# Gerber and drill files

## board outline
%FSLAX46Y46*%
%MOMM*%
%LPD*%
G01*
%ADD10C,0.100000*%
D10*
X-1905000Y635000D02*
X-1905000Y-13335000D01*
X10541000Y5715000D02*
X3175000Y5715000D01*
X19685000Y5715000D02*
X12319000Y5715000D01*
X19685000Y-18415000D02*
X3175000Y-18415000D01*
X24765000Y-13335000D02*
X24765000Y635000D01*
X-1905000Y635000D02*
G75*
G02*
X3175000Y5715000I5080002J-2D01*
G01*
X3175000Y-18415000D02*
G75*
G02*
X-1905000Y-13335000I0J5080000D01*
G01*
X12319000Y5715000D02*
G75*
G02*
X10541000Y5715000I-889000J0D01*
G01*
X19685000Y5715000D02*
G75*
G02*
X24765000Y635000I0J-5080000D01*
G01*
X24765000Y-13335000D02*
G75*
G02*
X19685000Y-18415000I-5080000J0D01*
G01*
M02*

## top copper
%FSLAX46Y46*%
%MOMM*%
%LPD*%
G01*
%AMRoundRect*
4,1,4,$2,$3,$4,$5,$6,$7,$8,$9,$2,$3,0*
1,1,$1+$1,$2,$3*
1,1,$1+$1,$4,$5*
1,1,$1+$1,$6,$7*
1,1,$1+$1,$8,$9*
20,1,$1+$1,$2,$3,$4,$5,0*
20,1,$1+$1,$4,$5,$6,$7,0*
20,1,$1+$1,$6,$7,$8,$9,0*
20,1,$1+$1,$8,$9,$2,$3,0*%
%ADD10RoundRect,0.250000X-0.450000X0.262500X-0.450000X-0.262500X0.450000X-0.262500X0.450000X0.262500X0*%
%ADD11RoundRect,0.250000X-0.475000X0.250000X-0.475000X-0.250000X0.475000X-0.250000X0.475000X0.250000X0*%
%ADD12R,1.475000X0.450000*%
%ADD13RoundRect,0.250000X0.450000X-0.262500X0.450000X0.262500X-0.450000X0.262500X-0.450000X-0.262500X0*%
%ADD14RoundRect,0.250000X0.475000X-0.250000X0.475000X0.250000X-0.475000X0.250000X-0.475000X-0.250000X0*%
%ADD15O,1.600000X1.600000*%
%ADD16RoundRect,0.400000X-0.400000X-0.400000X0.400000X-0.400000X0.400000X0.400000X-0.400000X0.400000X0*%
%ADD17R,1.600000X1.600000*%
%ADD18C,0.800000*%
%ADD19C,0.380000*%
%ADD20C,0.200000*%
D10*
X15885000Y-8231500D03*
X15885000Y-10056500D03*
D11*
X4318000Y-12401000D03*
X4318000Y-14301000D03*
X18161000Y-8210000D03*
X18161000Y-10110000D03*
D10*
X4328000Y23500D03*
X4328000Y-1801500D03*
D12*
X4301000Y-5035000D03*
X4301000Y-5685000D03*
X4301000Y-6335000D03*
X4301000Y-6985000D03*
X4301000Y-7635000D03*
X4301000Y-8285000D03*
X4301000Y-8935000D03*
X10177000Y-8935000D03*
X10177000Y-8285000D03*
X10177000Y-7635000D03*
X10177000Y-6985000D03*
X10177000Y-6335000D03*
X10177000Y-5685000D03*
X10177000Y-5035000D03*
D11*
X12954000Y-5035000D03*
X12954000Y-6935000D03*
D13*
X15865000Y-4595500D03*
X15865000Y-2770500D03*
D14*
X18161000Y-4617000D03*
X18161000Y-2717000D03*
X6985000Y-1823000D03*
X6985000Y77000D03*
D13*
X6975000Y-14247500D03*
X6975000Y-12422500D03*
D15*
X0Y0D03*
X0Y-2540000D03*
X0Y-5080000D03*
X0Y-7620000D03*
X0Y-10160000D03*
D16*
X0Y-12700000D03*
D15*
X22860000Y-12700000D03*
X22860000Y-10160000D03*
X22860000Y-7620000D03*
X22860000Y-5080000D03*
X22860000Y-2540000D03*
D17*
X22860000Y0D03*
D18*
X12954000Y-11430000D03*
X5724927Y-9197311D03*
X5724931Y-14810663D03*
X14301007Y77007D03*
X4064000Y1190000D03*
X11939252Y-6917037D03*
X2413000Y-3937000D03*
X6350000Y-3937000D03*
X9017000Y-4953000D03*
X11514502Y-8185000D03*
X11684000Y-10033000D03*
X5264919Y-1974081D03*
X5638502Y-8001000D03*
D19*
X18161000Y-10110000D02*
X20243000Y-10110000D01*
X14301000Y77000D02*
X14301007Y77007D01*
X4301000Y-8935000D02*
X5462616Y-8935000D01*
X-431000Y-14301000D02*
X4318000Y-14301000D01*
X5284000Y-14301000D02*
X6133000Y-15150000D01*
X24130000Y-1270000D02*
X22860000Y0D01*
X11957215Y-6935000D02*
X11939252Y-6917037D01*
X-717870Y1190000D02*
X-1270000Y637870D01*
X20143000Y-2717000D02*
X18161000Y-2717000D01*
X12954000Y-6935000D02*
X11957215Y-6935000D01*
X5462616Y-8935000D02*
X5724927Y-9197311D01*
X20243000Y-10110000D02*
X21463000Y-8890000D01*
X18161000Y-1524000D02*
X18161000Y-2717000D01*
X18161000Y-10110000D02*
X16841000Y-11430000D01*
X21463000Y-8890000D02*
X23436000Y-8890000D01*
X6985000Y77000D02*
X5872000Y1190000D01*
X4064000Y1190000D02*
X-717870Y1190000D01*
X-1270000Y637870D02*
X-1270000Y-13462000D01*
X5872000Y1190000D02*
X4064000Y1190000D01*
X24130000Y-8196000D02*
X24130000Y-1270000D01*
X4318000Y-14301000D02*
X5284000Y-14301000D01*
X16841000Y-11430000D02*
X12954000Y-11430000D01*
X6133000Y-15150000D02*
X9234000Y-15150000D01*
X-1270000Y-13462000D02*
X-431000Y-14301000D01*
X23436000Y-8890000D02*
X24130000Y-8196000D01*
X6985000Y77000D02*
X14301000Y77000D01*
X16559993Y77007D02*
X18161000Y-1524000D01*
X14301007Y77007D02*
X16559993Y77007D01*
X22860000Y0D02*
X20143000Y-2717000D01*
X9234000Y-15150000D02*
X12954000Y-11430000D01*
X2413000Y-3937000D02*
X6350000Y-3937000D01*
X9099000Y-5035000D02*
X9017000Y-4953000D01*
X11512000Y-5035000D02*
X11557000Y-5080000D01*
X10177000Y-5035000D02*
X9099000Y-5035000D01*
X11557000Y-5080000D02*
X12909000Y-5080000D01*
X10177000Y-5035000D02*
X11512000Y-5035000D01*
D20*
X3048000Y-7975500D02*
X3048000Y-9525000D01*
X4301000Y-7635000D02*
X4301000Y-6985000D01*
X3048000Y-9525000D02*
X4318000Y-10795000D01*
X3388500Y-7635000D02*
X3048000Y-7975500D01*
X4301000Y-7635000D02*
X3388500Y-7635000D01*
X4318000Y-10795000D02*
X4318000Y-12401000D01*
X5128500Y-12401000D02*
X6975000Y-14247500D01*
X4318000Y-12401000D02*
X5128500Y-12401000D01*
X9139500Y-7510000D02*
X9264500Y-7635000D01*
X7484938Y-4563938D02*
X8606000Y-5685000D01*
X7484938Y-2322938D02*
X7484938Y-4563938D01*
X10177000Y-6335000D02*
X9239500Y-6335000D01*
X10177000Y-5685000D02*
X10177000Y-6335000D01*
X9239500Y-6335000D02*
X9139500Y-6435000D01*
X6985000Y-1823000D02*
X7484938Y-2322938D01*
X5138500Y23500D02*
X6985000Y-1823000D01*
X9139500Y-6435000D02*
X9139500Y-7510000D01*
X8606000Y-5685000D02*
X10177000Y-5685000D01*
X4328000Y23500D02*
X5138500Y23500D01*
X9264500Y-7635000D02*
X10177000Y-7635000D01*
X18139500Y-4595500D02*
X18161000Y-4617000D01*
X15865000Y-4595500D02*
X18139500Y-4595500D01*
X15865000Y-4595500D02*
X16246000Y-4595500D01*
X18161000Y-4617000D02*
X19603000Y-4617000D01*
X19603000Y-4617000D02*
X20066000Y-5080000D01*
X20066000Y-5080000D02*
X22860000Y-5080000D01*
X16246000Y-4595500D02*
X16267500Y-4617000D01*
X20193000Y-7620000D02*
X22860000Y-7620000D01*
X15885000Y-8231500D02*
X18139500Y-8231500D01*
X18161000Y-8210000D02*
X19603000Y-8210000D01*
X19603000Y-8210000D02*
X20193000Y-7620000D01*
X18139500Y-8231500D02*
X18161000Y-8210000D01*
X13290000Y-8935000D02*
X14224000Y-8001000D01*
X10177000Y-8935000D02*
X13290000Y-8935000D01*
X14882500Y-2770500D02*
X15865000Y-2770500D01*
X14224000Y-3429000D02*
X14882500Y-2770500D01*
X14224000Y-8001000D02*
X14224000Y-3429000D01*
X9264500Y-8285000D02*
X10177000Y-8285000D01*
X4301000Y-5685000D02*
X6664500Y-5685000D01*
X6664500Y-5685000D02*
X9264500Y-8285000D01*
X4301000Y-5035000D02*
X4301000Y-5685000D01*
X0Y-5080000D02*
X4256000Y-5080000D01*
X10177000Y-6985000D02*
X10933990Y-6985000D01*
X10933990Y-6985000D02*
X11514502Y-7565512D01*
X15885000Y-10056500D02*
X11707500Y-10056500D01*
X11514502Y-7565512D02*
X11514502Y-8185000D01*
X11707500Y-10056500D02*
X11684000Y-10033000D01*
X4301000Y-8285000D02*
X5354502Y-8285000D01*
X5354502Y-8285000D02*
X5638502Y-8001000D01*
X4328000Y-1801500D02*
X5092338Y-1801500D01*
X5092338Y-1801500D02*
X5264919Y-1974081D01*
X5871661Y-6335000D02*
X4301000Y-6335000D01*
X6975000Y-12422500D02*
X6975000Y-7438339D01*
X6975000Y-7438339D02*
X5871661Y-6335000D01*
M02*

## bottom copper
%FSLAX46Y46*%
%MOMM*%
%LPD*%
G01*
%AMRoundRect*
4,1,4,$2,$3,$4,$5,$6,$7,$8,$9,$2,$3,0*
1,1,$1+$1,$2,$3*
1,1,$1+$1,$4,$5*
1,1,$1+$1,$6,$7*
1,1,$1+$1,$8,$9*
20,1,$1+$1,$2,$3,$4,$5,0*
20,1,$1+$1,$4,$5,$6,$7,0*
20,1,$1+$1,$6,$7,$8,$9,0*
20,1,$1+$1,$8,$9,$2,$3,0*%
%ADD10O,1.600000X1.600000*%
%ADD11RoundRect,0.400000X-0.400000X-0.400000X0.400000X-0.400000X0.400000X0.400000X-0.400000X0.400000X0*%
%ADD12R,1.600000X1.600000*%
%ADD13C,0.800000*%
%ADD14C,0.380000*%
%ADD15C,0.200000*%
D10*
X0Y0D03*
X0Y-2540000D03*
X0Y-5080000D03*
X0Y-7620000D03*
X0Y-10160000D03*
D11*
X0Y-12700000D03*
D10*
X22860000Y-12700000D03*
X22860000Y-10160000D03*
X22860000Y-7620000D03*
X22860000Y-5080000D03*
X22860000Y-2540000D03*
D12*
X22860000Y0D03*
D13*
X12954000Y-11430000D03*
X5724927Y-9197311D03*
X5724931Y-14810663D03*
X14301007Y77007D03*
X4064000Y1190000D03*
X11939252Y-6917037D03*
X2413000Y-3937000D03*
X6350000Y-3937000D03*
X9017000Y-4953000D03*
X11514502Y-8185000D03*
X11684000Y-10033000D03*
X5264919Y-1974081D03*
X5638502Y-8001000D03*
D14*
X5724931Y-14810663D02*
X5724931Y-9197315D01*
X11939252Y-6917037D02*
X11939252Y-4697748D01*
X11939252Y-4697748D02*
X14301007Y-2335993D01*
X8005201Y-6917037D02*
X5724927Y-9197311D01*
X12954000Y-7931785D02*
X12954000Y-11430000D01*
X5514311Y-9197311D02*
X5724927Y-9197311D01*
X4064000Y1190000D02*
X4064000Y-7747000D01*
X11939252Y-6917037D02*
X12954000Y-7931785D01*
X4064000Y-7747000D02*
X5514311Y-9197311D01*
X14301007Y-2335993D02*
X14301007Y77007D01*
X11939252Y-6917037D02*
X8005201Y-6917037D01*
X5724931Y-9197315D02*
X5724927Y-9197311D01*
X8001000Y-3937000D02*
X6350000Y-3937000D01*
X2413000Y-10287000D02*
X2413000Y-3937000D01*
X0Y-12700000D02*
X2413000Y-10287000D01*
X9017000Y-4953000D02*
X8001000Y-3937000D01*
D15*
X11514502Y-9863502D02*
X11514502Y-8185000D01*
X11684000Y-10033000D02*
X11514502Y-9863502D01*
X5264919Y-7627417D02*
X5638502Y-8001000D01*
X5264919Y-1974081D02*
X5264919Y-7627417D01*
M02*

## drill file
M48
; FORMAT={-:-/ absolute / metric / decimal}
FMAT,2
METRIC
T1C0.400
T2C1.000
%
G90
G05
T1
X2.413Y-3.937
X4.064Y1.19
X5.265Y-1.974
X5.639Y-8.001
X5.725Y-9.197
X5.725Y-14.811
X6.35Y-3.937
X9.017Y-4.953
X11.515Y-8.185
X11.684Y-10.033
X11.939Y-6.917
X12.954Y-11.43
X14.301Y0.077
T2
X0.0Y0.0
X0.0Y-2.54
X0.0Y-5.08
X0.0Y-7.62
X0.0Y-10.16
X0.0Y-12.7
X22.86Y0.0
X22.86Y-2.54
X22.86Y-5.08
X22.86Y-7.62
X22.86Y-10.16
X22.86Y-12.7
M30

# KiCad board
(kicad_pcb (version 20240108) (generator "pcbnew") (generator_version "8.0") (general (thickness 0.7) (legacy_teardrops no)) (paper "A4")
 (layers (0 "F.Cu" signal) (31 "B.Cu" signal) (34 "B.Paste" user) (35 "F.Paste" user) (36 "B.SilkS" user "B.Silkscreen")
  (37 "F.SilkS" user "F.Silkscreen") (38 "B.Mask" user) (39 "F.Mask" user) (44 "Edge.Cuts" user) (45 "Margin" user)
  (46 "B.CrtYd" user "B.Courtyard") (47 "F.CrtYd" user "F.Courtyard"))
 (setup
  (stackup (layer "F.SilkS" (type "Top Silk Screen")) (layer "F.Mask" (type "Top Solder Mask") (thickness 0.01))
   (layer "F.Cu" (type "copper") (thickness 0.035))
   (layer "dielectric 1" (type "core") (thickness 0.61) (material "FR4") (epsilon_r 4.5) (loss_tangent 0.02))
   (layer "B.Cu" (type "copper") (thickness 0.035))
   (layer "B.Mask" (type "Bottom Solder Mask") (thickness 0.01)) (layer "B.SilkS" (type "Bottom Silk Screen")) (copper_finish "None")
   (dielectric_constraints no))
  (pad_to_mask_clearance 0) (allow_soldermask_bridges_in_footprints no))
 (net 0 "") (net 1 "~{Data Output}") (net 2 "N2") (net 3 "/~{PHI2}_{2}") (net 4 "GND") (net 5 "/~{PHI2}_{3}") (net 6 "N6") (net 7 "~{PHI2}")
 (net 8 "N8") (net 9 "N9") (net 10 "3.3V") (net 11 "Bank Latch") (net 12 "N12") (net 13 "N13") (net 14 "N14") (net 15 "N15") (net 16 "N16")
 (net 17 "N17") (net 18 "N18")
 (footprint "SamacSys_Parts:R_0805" (layer "F.Cu") (at 15.875 9.144 180)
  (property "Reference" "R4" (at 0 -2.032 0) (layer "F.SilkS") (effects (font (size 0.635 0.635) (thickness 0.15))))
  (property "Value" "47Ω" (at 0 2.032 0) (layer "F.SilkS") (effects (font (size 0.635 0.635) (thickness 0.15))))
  (pad "1" smd roundrect (at -0.01 0.9125 270) (size 1.025 1.4) (layers "F.Cu" "F.Paste" "F.Mask") (roundrect_rratio 0.243902)
   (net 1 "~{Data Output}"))
  (pad "2" smd roundrect (at -0.01 -0.9125 270) (size 1.025 1.4) (layers "F.Cu" "F.Paste" "F.Mask") (roundrect_rratio 0.243902) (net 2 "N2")))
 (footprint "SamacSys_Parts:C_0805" (layer "F.Cu") (at 4.318 13.335 180)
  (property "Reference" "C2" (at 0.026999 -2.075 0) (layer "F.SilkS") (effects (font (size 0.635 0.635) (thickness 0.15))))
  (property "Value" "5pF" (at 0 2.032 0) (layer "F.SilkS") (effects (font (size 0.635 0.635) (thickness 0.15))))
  (pad "1" smd roundrect (at 0 0.934 270) (size 1 1.45) (layers "F.Cu" "F.Paste" "F.Mask") (roundrect_rratio 0.25) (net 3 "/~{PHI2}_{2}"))
  (pad "2" smd roundrect (at 0 -0.966 270) (size 1 1.45) (layers "F.Cu" "F.Paste" "F.Mask") (roundrect_rratio 0.25) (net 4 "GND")))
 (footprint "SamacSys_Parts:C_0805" (layer "F.Cu") (at 18.161 9.144 180)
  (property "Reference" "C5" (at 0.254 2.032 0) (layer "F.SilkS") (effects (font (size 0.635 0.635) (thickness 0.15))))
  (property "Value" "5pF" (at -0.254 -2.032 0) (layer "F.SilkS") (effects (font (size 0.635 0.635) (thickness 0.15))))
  (pad "1" smd roundrect (at 0 0.934 270) (size 1 1.45) (layers "F.Cu" "F.Paste" "F.Mask") (roundrect_rratio 0.25) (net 1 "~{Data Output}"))
  (pad "2" smd roundrect (at 0 -0.966 270) (size 1 1.45) (layers "F.Cu" "F.Paste" "F.Mask") (roundrect_rratio 0.25) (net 4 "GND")))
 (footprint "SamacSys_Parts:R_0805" (layer "F.Cu") (at 4.318 0.889 180)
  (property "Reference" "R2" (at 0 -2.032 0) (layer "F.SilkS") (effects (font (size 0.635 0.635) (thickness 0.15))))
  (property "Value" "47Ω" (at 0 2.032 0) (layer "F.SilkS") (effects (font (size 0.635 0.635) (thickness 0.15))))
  (pad "1" smd roundrect (at -0.01 0.9125 270) (size 1.025 1.4) (layers "F.Cu" "F.Paste" "F.Mask") (roundrect_rratio 0.243902)
   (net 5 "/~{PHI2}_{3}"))
  (pad "2" smd roundrect (at -0.01 -0.9125 270) (size 1.025 1.4) (layers "F.Cu" "F.Paste" "F.Mask") (roundrect_rratio 0.243902) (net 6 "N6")))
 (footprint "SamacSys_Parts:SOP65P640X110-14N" (layer "F.Cu") (at 7.239 6.985)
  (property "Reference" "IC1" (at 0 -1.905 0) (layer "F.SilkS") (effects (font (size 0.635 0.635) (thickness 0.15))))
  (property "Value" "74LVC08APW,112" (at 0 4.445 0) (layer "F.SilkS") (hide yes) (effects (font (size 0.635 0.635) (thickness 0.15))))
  (pad "1" smd rect (at -2.938 -1.95 90) (size 0.45 1.475) (layers "F.Cu" "F.Paste" "F.Mask") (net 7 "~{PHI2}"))
  (pad "2" smd rect (at -2.938 -1.3 90) (size 0.45 1.475) (layers "F.Cu" "F.Paste" "F.Mask") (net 7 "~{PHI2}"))
  (pad "3" smd rect (at -2.938 -0.65 90) (size 0.45 1.475) (layers "F.Cu" "F.Paste" "F.Mask") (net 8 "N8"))
  (pad "4" smd rect (at -2.938 0 90) (size 0.45 1.475) (layers "F.Cu" "F.Paste" "F.Mask") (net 3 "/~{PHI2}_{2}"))
  (pad "5" smd rect (at -2.938 0.65 90) (size 0.45 1.475) (layers "F.Cu" "F.Paste" "F.Mask") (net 3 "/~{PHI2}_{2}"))
  (pad "6" smd rect (at -2.938 1.3 90) (size 0.45 1.475) (layers "F.Cu" "F.Paste" "F.Mask") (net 6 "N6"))
  (pad "7" smd rect (at -2.938 1.95 90) (size 0.45 1.475) (layers "F.Cu" "F.Paste" "F.Mask") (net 4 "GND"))
  (pad "8" smd rect (at 2.938 1.95 90) (size 0.45 1.475) (layers "F.Cu" "F.Paste" "F.Mask") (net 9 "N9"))
  (pad "9" smd rect (at 2.938 1.3 90) (size 0.45 1.475) (layers "F.Cu" "F.Paste" "F.Mask") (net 7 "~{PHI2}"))
  (pad "10" smd rect (at 2.938 0.65 90) (size 0.45 1.475) (layers "F.Cu" "F.Paste" "F.Mask") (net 5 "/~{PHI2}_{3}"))
  (pad "11" smd rect (at 2.938 0 90) (size 0.45 1.475) (layers "F.Cu" "F.Paste" "F.Mask") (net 2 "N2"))
  (pad "12" smd rect (at 2.938 -0.65 90) (size 0.45 1.475) (layers "F.Cu" "F.Paste" "F.Mask") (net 5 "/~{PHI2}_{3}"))
  (pad "13" smd rect (at 2.938 -1.3 90) (size 0.45 1.475) (layers "F.Cu" "F.Paste" "F.Mask") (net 5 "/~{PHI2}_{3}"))
  (pad "14" smd rect (at 2.938 -1.95 90) (size 0.45 1.475) (layers "F.Cu" "F.Paste" "F.Mask") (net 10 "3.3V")))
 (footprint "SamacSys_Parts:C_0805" (layer "F.Cu") (at 12.954 5.969 180)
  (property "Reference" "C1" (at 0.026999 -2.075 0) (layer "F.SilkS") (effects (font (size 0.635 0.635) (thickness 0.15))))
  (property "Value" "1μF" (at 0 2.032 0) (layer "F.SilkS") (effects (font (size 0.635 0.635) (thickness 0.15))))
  (pad "1" smd roundrect (at 0 0.934 270) (size 1 1.45) (layers "F.Cu" "F.Paste" "F.Mask") (roundrect_rratio 0.25) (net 10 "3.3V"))
  (pad "2" smd roundrect (at 0 -0.966 270) (size 1 1.45) (layers "F.Cu" "F.Paste" "F.Mask") (roundrect_rratio 0.25) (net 4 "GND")))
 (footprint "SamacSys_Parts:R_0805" (layer "F.Cu") (at 15.875 3.683)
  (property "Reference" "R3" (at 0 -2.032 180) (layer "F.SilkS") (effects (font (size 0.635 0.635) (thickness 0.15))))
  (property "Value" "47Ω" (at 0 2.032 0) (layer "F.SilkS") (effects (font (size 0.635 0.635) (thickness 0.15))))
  (pad "1" smd roundrect (at -0.01 0.9125 90) (size 1.025 1.4) (layers "F.Cu" "F.Paste" "F.Mask") (roundrect_rratio 0.243902)
   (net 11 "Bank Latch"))
  (pad "2" smd roundrect (at -0.01 -0.9125 90) (size 1.025 1.4) (layers "F.Cu" "F.Paste" "F.Mask") (roundrect_rratio 0.243902) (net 9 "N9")))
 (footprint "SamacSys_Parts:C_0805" (layer "F.Cu") (at 18.161 3.683)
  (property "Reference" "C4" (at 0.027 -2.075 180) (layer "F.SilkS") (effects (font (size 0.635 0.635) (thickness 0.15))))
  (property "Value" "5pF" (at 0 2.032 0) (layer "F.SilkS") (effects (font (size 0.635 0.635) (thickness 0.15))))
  (pad "1" smd roundrect (at 0 0.934 90) (size 1 1.45) (layers "F.Cu" "F.Paste" "F.Mask") (roundrect_rratio 0.25) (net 11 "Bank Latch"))
  (pad "2" smd roundrect (at 0 -0.966 90) (size 1 1.45) (layers "F.Cu" "F.Paste" "F.Mask") (roundrect_rratio 0.25) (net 4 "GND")))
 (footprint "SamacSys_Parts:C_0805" (layer "F.Cu") (at 6.985 0.889)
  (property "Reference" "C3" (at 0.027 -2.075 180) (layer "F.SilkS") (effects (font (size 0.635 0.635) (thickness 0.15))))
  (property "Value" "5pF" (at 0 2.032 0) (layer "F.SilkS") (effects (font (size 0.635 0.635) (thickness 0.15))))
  (pad "1" smd roundrect (at 0 0.934 90) (size 1 1.45) (layers "F.Cu" "F.Paste" "F.Mask") (roundrect_rratio 0.25) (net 5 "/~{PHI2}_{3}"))
  (pad "2" smd roundrect (at 0 -0.966 90) (size 1 1.45) (layers "F.Cu" "F.Paste" "F.Mask") (roundrect_rratio 0.25) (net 4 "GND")))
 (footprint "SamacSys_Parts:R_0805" (layer "F.Cu") (at 6.985 13.335)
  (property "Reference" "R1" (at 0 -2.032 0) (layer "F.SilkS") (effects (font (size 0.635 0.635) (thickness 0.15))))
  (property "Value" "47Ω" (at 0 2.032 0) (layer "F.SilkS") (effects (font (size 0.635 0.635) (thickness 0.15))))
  (pad "1" smd roundrect (at -0.01 0.9125 90) (size 1.025 1.4) (layers "F.Cu" "F.Paste" "F.Mask") (roundrect_rratio 0.243902)
   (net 3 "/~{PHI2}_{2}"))
  (pad "2" smd roundrect (at -0.01 -0.9125 90) (size 1.025 1.4) (layers "F.Cu" "F.Paste" "F.Mask") (roundrect_rratio 0.243902) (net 8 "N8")))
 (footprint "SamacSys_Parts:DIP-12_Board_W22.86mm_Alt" (layer "F.Cu") (at 0 0)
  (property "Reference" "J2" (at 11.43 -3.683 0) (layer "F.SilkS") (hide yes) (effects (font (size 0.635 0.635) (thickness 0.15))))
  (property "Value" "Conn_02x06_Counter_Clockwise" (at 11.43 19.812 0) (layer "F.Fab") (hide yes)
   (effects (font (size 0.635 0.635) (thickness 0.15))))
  (fp_line (start -1.905 -0.635) (end -1.905 13.335) (stroke (width 0.1) (type solid)) (layer "Edge.Cuts"))
  (fp_line (start 10.541 -5.715) (end 3.175 -5.715) (stroke (width 0.1) (type solid)) (layer "Edge.Cuts"))
  (fp_line (start 19.685 -5.715) (end 12.319 -5.715) (stroke (width 0.1) (type solid)) (layer "Edge.Cuts"))
  (fp_line (start 19.685 18.415) (end 3.175 18.415) (stroke (width 0.1) (type solid)) (layer "Edge.Cuts"))
  (fp_line (start 24.765 13.335) (end 24.765 -0.635) (stroke (width 0.1) (type solid)) (layer "Edge.Cuts"))
  (fp_arc (start -1.905 -0.635) (mid -0.417102 -4.227102) (end 3.175 -5.715) (stroke (width 0.1) (type solid)) (layer "Edge.Cuts"))
  (fp_arc (start 3.175 18.415) (mid -0.417102 16.927102) (end -1.905 13.335) (stroke (width 0.1) (type solid)) (layer "Edge.Cuts"))
  (fp_arc (start 12.319 -5.715) (mid 11.43 -4.826) (end 10.541 -5.715) (stroke (width 0.1) (type default)) (layer "Edge.Cuts"))
  (fp_arc (start 19.685 -5.715) (mid 23.277102 -4.227102) (end 24.765 -0.635) (stroke (width 0.1) (type solid)) (layer "Edge.Cuts"))
  (fp_arc (start 24.765 13.335) (mid 23.277102 16.927102) (end 19.685 18.415) (stroke (width 0.1) (type solid)) (layer "Edge.Cuts"))
  (pad "1" thru_hole oval (at 0 0) (size 1.6 1.6) (drill 1) (layers "*.Cu" "*.Mask") (remove_unused_layers no) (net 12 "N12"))
  (pad "2" thru_hole oval (at 0 2.54) (size 1.6 1.6) (drill 1) (layers "*.Cu" "*.Mask") (remove_unused_layers no) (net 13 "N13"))
  (pad "3" thru_hole oval (at 0 5.08) (size 1.6 1.6) (drill 1) (layers "*.Cu" "*.Mask") (remove_unused_layers no) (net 7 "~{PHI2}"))
  (pad "4" thru_hole oval (at 0 7.62) (size 1.6 1.6) (drill 1) (layers "*.Cu" "*.Mask") (remove_unused_layers no) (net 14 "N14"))
  (pad "5" thru_hole oval (at 0 10.16) (size 1.6 1.6) (drill 1) (layers "*.Cu" "*.Mask") (remove_unused_layers no) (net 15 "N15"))
  (pad "6" thru_hole roundrect (at 0 12.7) (size 1.6 1.6) (drill 1) (layers "*.Cu" "*.Mask") (remove_unused_layers no)
   (roundrect_rratio 0.25) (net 10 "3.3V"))
  (pad "7" thru_hole oval (at 22.86 12.7 180) (size 1.6 1.6) (drill 1) (layers "*.Cu" "*.Mask") (remove_unused_layers no) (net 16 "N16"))
  (pad "8" thru_hole oval (at 22.86 10.16 180) (size 1.6 1.6) (drill 1) (layers "*.Cu" "*.Mask") (remove_unused_layers no) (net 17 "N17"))
  (pad "9" thru_hole oval (at 22.86 7.62) (size 1.6 1.6) (drill 1) (layers "*.Cu" "*.Mask") (remove_unused_layers no)
   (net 1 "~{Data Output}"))
  (pad "10" thru_hole oval (at 22.86 5.08) (size 1.6 1.6) (drill 1) (layers "*.Cu" "*.Mask") (remove_unused_layers no) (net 11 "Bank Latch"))
  (pad "11" thru_hole oval (at 22.86 2.54) (size 1.6 1.6) (drill 1) (layers "*.Cu" "*.Mask") (remove_unused_layers no) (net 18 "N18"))
  (pad "12" thru_hole rect (at 22.86 0) (size 1.6 1.6) (drill 1) (layers "*.Cu" "*.Mask") (remove_unused_layers no) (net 4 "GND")))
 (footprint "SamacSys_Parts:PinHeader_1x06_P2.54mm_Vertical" (layer "B.Cu") (at 22.86 0 180)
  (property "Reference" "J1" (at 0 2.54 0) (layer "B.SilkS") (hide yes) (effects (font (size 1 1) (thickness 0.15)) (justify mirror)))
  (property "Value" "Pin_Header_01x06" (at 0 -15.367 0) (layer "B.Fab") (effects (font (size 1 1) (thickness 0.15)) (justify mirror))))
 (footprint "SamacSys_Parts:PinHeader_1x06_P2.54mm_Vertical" (layer "B.Cu") (at 0 0 180)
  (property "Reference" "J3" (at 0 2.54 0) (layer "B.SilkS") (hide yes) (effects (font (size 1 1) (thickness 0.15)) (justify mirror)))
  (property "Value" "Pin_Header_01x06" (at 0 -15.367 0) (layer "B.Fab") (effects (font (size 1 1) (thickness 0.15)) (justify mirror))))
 (segment (start 18.161 10.11) (end 20.243 10.11) (width 0.38) (layer "F.Cu") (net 4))
 (segment (start 14.301 -0.077) (end 14.301007 -0.077007) (width 0.38) (layer "F.Cu") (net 4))
 (segment (start 4.301 8.935) (end 5.462616 8.935) (width 0.38) (layer "F.Cu") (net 4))
 (segment (start -0.431 14.301) (end 4.318 14.301) (width 0.38) (layer "F.Cu") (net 4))
 (segment (start 5.284 14.301) (end 6.133 15.15) (width 0.38) (layer "F.Cu") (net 4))
 (segment (start 24.13 1.27) (end 22.86 0) (width 0.38) (layer "F.Cu") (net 4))
 (segment (start 11.957215 6.935) (end 11.939252 6.917037) (width 0.38) (layer "F.Cu") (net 4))
 (segment (start -0.71787 -1.19) (end -1.27 -0.63787) (width 0.38) (layer "F.Cu") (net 4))
 (segment (start 20.143 2.717) (end 18.161 2.717) (width 0.38) (layer "F.Cu") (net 4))
 (segment (start 12.954 6.935) (end 11.957215 6.935) (width 0.38) (layer "F.Cu") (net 4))
 (segment (start 5.462616 8.935) (end 5.724927 9.197311) (width 0.38) (layer "F.Cu") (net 4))
 (segment (start 20.243 10.11) (end 21.463 8.89) (width 0.38) (layer "F.Cu") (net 4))
 (segment (start 18.161 1.524) (end 18.161 2.717) (width 0.38) (layer "F.Cu") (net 4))
 (segment (start 18.161 10.11) (end 16.841 11.43) (width 0.38) (layer "F.Cu") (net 4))
 (segment (start 21.463 8.89) (end 23.436 8.89) (width 0.38) (layer "F.Cu") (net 4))
 (segment (start 6.985 -0.077) (end 5.872 -1.19) (width 0.38) (layer "F.Cu") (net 4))
 (segment (start 4.064 -1.19) (end -0.71787 -1.19) (width 0.38) (layer "F.Cu") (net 4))
 (segment (start -1.27 -0.63787) (end -1.27 13.462) (width 0.38) (layer "F.Cu") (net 4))
 (segment (start 5.872 -1.19) (end 4.064 -1.19) (width 0.38) (layer "F.Cu") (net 4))
 (segment (start 24.13 8.196) (end 24.13 1.27) (width 0.38) (layer "F.Cu") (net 4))
 (segment (start 4.318 14.301) (end 5.284 14.301) (width 0.38) (layer "F.Cu") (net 4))
 (segment (start 16.841 11.43) (end 12.954 11.43) (width 0.38) (layer "F.Cu") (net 4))
 (segment (start 6.133 15.15) (end 9.234 15.15) (width 0.38) (layer "F.Cu") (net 4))
 (segment (start -1.27 13.462) (end -0.431 14.301) (width 0.38) (layer "F.Cu") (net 4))
 (segment (start 23.436 8.89) (end 24.13 8.196) (width 0.38) (layer "F.Cu") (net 4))
 (segment (start 6.985 -0.077) (end 14.301 -0.077) (width 0.38) (layer "F.Cu") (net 4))
 (segment (start 16.559993 -0.077007) (end 18.161 1.524) (width 0.38) (layer "F.Cu") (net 4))
 (segment (start 14.301007 -0.077007) (end 16.559993 -0.077007) (width 0.38) (layer "F.Cu") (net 4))
 (segment (start 22.86 0) (end 20.143 2.717) (width 0.38) (layer "F.Cu") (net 4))
 (segment (start 9.234 15.15) (end 12.954 11.43) (width 0.38) (layer "F.Cu") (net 4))
 (via (at 12.954 11.43) (size 0.8) (drill 0.4) (layers "F.Cu" "B.Cu") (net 4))
 (via (at 5.724927 9.197311) (size 0.8) (drill 0.4) (layers "F.Cu" "B.Cu") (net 4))
 (via (at 5.724931 14.810663) (size 0.8) (drill 0.4) (layers "F.Cu" "B.Cu") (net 4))
 (via (at 14.301007 -0.077007) (size 0.8) (drill 0.4) (layers "F.Cu" "B.Cu") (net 4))
 (via (at 4.064 -1.19) (size 0.8) (drill 0.4) (layers "F.Cu" "B.Cu") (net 4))
 (via (at 11.939252 6.917037) (size 0.8) (drill 0.4) (layers "F.Cu" "B.Cu") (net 4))
 (segment (start 5.724931 14.810663) (end 5.724931 9.197315) (width 0.38) (layer "B.Cu") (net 4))
 (segment (start 11.939252 6.917037) (end 11.939252 4.697748) (width 0.38) (layer "B.Cu") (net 4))
 (segment (start 11.939252 4.697748) (end 14.301007 2.335993) (width 0.38) (layer "B.Cu") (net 4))
 (segment (start 8.005201 6.917037) (end 5.724927 9.197311) (width 0.38) (layer "B.Cu") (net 4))
 (segment (start 12.954 7.931785) (end 12.954 11.43) (width 0.38) (layer "B.Cu") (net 4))
 (segment (start 5.514311 9.197311) (end 5.724927 9.197311) (width 0.38) (layer "B.Cu") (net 4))
 (segment (start 4.064 -1.19) (end 4.064 7.747) (width 0.38) (layer "B.Cu") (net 4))
 (segment (start 11.939252 6.917037) (end 12.954 7.931785) (width 0.38) (layer "B.Cu") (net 4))
 (segment (start 4.064 7.747) (end 5.514311 9.197311) (width 0.38) (layer "B.Cu") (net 4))
 (segment (start 14.301007 2.335993) (end 14.301007 -0.077007) (width 0.38) (layer "B.Cu") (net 4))
 (segment (start 11.939252 6.917037) (end 8.005201 6.917037) (width 0.38) (layer "B.Cu") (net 4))
 (segment (start 5.724931 9.197315) (end 5.724927 9.197311) (width 0.38) (layer "B.Cu") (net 4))
 (segment (start 2.413 3.937) (end 6.35 3.937) (width 0.38) (layer "F.Cu") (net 10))
 (segment (start 9.099 5.035) (end 9.017 4.953) (width 0.38) (layer "F.Cu") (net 10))
 (segment (start 11.512 5.035) (end 11.557 5.08) (width 0.38) (layer "F.Cu") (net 10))
 (segment (start 10.177 5.035) (end 9.099 5.035) (width 0.38) (layer "F.Cu") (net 10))
 (segment (start 11.557 5.08) (end 12.909 5.08) (width 0.38) (layer "F.Cu") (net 10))
 (segment (start 10.177 5.035) (end 11.512 5.035) (width 0.38) (layer "F.Cu") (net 10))
 (via (at 2.413 3.937) (size 0.8) (drill 0.4) (layers "F.Cu" "B.Cu") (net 10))
 (via (at 6.35 3.937) (size 0.8) (drill 0.4) (layers "F.Cu" "B.Cu") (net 10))
 (via (at 9.017 4.953) (size 0.8) (drill 0.4) (layers "F.Cu" "B.Cu") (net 10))
 (segment (start 8.001 3.937) (end 6.35 3.937) (width 0.38) (layer "B.Cu") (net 10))
 (segment (start 2.413 10.287) (end 2.413 3.937) (width 0.38) (layer "B.Cu") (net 10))
 (segment (start 0 12.7) (end 2.413 10.287) (width 0.38) (layer "B.Cu") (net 10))
 (segment (start 9.017 4.953) (end 8.001 3.937) (width 0.38) (layer "B.Cu") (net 10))
 (segment (start 3.048 7.9755) (end 3.048 9.525) (width 0.2) (layer "F.Cu") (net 3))
 (segment (start 4.301 7.635) (end 4.301 6.985) (width 0.2) (layer "F.Cu") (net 3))
 (segment (start 3.048 9.525) (end 4.318 10.795) (width 0.2) (layer "F.Cu") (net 3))
 (segment (start 3.3885 7.635) (end 3.048 7.9755) (width 0.2) (layer "F.Cu") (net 3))
 (segment (start 4.301 7.635) (end 3.3885 7.635) (width 0.2) (layer "F.Cu") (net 3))
 (segment (start 4.318 10.795) (end 4.318 12.401) (width 0.2) (layer "F.Cu") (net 3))
 (segment (start 5.1285 12.401) (end 6.975 14.2475) (width 0.2) (layer "F.Cu") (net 3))
 (segment (start 4.318 12.401) (end 5.1285 12.401) (width 0.2) (layer "F.Cu") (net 3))
 (segment (start 9.1395 7.51) (end 9.2645 7.635) (width 0.2) (layer "F.Cu") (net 5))
 (segment (start 7.484938 4.563938) (end 8.606 5.685) (width 0.2) (layer "F.Cu") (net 5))
 (segment (start 7.484938 2.322938) (end 7.484938 4.563938) (width 0.2) (layer "F.Cu") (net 5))
 (segment (start 10.177 6.335) (end 9.2395 6.335) (width 0.2) (layer "F.Cu") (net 5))
 (segment (start 10.177 5.685) (end 10.177 6.335) (width 0.2) (layer "F.Cu") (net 5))
 (segment (start 9.2395 6.335) (end 9.1395 6.435) (width 0.2) (layer "F.Cu") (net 5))
 (segment (start 6.985 1.823) (end 7.484938 2.322938) (width 0.2) (layer "F.Cu") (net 5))
 (segment (start 5.1385 -0.0235) (end 6.985 1.823) (width 0.2) (layer "F.Cu") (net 5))
 (segment (start 9.1395 6.435) (end 9.1395 7.51) (width 0.2) (layer "F.Cu") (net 5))
 (segment (start 8.606 5.685) (end 10.177 5.685) (width 0.2) (layer "F.Cu") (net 5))
 (segment (start 4.328 -0.0235) (end 5.1385 -0.0235) (width 0.2) (layer "F.Cu") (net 5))
 (segment (start 9.2645 7.635) (end 10.177 7.635) (width 0.2) (layer "F.Cu") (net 5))
 (segment (start 18.1395 4.5955) (end 18.161 4.617) (width 0.2) (layer "F.Cu") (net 11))
 (segment (start 15.865 4.5955) (end 18.1395 4.5955) (width 0.2) (layer "F.Cu") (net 11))
 (segment (start 15.865 4.5955) (end 16.246 4.5955) (width 0.2) (layer "F.Cu") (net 11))
 (segment (start 18.161 4.617) (end 19.603 4.617) (width 0.2) (layer "F.Cu") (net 11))
 (segment (start 19.603 4.617) (end 20.066 5.08) (width 0.2) (layer "F.Cu") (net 11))
 (segment (start 20.066 5.08) (end 22.86 5.08) (width 0.2) (layer "F.Cu") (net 11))
 (segment (start 16.246 4.5955) (end 16.2675 4.617) (width 0.2) (layer "F.Cu") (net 11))
 (segment (start 20.193 7.62) (end 22.86 7.62) (width 0.2) (layer "F.Cu") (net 1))
 (segment (start 15.885 8.2315) (end 18.1395 8.2315) (width 0.2) (layer "F.Cu") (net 1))
 (segment (start 18.161 8.21) (end 19.603 8.21) (width 0.2) (layer "F.Cu") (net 1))
 (segment (start 19.603 8.21) (end 20.193 7.62) (width 0.2) (layer "F.Cu") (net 1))
 (segment (start 18.1395 8.2315) (end 18.161 8.21) (width 0.2) (layer "F.Cu") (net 1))
 (segment (start 13.29 8.935) (end 14.224 8.001) (width 0.2) (layer "F.Cu") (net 9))
 (segment (start 10.177 8.935) (end 13.29 8.935) (width 0.2) (layer "F.Cu") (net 9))
 (segment (start 14.8825 2.7705) (end 15.865 2.7705) (width 0.2) (layer "F.Cu") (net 9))
 (segment (start 14.224 3.429) (end 14.8825 2.7705) (width 0.2) (layer "F.Cu") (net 9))
 (segment (start 14.224 8.001) (end 14.224 3.429) (width 0.2) (layer "F.Cu") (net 9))
 (segment (start 9.2645 8.285) (end 10.177 8.285) (width 0.2) (layer "F.Cu") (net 7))
 (segment (start 4.301 5.685) (end 6.6645 5.685) (width 0.2) (layer "F.Cu") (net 7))
 (segment (start 6.6645 5.685) (end 9.2645 8.285) (width 0.2) (layer "F.Cu") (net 7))
 (segment (start 4.301 5.035) (end 4.301 5.685) (width 0.2) (layer "F.Cu") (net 7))
 (segment (start 0 5.08) (end 4.256 5.08) (width 0.2) (layer "F.Cu") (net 7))
 (segment (start 10.177 6.985) (end 10.93399 6.985) (width 0.2) (layer "F.Cu") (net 2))
 (segment (start 10.93399 6.985) (end 11.514502 7.565512) (width 0.2) (layer "F.Cu") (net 2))
 (segment (start 15.885 10.0565) (end 11.7075 10.0565) (width 0.2) (layer "F.Cu") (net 2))
 (segment (start 11.514502 7.565512) (end 11.514502 8.185) (width 0.2) (layer "F.Cu") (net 2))
 (segment (start 11.7075 10.0565) (end 11.684 10.033) (width 0.2) (layer "F.Cu") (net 2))
 (via (at 11.514502 8.185) (size 0.8) (drill 0.4) (layers "F.Cu" "B.Cu") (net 2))
 (via (at 11.684 10.033) (size 0.8) (drill 0.4) (layers "F.Cu" "B.Cu") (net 2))
 (segment (start 11.514502 9.863502) (end 11.514502 8.185) (width 0.2) (layer "B.Cu") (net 2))
 (segment (start 11.684 10.033) (end 11.514502 9.863502) (width 0.2) (layer "B.Cu") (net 2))
 (segment (start 4.301 8.285) (end 5.354502 8.285) (width 0.2) (layer "F.Cu") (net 6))
 (segment (start 5.354502 8.285) (end 5.638502 8.001) (width 0.2) (layer "F.Cu") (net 6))
 (segment (start 4.328 1.8015) (end 5.092338 1.8015) (width 0.2) (layer "F.Cu") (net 6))
 (segment (start 5.092338 1.8015) (end 5.264919 1.974081) (width 0.2) (layer "F.Cu") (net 6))
 (via (at 5.264919 1.974081) (size 0.8) (drill 0.4) (layers "F.Cu" "B.Cu") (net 6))
 (via (at 5.638502 8.001) (size 0.8) (drill 0.4) (layers "F.Cu" "B.Cu") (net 6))
 (segment (start 5.264919 7.627417) (end 5.638502 8.001) (width 0.2) (layer "B.Cu") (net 6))
 (segment (start 5.264919 1.974081) (end 5.264919 7.627417) (width 0.2) (layer "B.Cu") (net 6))
 (segment (start 5.871661 6.335) (end 4.301 6.335) (width 0.2) (layer "F.Cu") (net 8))
 (segment (start 6.975 12.4225) (end 6.975 7.438339) (width 0.2) (layer "F.Cu") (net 8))
 (segment (start 6.975 7.438339) (end 5.871661 6.335) (width 0.2) (layer "F.Cu") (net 8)))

